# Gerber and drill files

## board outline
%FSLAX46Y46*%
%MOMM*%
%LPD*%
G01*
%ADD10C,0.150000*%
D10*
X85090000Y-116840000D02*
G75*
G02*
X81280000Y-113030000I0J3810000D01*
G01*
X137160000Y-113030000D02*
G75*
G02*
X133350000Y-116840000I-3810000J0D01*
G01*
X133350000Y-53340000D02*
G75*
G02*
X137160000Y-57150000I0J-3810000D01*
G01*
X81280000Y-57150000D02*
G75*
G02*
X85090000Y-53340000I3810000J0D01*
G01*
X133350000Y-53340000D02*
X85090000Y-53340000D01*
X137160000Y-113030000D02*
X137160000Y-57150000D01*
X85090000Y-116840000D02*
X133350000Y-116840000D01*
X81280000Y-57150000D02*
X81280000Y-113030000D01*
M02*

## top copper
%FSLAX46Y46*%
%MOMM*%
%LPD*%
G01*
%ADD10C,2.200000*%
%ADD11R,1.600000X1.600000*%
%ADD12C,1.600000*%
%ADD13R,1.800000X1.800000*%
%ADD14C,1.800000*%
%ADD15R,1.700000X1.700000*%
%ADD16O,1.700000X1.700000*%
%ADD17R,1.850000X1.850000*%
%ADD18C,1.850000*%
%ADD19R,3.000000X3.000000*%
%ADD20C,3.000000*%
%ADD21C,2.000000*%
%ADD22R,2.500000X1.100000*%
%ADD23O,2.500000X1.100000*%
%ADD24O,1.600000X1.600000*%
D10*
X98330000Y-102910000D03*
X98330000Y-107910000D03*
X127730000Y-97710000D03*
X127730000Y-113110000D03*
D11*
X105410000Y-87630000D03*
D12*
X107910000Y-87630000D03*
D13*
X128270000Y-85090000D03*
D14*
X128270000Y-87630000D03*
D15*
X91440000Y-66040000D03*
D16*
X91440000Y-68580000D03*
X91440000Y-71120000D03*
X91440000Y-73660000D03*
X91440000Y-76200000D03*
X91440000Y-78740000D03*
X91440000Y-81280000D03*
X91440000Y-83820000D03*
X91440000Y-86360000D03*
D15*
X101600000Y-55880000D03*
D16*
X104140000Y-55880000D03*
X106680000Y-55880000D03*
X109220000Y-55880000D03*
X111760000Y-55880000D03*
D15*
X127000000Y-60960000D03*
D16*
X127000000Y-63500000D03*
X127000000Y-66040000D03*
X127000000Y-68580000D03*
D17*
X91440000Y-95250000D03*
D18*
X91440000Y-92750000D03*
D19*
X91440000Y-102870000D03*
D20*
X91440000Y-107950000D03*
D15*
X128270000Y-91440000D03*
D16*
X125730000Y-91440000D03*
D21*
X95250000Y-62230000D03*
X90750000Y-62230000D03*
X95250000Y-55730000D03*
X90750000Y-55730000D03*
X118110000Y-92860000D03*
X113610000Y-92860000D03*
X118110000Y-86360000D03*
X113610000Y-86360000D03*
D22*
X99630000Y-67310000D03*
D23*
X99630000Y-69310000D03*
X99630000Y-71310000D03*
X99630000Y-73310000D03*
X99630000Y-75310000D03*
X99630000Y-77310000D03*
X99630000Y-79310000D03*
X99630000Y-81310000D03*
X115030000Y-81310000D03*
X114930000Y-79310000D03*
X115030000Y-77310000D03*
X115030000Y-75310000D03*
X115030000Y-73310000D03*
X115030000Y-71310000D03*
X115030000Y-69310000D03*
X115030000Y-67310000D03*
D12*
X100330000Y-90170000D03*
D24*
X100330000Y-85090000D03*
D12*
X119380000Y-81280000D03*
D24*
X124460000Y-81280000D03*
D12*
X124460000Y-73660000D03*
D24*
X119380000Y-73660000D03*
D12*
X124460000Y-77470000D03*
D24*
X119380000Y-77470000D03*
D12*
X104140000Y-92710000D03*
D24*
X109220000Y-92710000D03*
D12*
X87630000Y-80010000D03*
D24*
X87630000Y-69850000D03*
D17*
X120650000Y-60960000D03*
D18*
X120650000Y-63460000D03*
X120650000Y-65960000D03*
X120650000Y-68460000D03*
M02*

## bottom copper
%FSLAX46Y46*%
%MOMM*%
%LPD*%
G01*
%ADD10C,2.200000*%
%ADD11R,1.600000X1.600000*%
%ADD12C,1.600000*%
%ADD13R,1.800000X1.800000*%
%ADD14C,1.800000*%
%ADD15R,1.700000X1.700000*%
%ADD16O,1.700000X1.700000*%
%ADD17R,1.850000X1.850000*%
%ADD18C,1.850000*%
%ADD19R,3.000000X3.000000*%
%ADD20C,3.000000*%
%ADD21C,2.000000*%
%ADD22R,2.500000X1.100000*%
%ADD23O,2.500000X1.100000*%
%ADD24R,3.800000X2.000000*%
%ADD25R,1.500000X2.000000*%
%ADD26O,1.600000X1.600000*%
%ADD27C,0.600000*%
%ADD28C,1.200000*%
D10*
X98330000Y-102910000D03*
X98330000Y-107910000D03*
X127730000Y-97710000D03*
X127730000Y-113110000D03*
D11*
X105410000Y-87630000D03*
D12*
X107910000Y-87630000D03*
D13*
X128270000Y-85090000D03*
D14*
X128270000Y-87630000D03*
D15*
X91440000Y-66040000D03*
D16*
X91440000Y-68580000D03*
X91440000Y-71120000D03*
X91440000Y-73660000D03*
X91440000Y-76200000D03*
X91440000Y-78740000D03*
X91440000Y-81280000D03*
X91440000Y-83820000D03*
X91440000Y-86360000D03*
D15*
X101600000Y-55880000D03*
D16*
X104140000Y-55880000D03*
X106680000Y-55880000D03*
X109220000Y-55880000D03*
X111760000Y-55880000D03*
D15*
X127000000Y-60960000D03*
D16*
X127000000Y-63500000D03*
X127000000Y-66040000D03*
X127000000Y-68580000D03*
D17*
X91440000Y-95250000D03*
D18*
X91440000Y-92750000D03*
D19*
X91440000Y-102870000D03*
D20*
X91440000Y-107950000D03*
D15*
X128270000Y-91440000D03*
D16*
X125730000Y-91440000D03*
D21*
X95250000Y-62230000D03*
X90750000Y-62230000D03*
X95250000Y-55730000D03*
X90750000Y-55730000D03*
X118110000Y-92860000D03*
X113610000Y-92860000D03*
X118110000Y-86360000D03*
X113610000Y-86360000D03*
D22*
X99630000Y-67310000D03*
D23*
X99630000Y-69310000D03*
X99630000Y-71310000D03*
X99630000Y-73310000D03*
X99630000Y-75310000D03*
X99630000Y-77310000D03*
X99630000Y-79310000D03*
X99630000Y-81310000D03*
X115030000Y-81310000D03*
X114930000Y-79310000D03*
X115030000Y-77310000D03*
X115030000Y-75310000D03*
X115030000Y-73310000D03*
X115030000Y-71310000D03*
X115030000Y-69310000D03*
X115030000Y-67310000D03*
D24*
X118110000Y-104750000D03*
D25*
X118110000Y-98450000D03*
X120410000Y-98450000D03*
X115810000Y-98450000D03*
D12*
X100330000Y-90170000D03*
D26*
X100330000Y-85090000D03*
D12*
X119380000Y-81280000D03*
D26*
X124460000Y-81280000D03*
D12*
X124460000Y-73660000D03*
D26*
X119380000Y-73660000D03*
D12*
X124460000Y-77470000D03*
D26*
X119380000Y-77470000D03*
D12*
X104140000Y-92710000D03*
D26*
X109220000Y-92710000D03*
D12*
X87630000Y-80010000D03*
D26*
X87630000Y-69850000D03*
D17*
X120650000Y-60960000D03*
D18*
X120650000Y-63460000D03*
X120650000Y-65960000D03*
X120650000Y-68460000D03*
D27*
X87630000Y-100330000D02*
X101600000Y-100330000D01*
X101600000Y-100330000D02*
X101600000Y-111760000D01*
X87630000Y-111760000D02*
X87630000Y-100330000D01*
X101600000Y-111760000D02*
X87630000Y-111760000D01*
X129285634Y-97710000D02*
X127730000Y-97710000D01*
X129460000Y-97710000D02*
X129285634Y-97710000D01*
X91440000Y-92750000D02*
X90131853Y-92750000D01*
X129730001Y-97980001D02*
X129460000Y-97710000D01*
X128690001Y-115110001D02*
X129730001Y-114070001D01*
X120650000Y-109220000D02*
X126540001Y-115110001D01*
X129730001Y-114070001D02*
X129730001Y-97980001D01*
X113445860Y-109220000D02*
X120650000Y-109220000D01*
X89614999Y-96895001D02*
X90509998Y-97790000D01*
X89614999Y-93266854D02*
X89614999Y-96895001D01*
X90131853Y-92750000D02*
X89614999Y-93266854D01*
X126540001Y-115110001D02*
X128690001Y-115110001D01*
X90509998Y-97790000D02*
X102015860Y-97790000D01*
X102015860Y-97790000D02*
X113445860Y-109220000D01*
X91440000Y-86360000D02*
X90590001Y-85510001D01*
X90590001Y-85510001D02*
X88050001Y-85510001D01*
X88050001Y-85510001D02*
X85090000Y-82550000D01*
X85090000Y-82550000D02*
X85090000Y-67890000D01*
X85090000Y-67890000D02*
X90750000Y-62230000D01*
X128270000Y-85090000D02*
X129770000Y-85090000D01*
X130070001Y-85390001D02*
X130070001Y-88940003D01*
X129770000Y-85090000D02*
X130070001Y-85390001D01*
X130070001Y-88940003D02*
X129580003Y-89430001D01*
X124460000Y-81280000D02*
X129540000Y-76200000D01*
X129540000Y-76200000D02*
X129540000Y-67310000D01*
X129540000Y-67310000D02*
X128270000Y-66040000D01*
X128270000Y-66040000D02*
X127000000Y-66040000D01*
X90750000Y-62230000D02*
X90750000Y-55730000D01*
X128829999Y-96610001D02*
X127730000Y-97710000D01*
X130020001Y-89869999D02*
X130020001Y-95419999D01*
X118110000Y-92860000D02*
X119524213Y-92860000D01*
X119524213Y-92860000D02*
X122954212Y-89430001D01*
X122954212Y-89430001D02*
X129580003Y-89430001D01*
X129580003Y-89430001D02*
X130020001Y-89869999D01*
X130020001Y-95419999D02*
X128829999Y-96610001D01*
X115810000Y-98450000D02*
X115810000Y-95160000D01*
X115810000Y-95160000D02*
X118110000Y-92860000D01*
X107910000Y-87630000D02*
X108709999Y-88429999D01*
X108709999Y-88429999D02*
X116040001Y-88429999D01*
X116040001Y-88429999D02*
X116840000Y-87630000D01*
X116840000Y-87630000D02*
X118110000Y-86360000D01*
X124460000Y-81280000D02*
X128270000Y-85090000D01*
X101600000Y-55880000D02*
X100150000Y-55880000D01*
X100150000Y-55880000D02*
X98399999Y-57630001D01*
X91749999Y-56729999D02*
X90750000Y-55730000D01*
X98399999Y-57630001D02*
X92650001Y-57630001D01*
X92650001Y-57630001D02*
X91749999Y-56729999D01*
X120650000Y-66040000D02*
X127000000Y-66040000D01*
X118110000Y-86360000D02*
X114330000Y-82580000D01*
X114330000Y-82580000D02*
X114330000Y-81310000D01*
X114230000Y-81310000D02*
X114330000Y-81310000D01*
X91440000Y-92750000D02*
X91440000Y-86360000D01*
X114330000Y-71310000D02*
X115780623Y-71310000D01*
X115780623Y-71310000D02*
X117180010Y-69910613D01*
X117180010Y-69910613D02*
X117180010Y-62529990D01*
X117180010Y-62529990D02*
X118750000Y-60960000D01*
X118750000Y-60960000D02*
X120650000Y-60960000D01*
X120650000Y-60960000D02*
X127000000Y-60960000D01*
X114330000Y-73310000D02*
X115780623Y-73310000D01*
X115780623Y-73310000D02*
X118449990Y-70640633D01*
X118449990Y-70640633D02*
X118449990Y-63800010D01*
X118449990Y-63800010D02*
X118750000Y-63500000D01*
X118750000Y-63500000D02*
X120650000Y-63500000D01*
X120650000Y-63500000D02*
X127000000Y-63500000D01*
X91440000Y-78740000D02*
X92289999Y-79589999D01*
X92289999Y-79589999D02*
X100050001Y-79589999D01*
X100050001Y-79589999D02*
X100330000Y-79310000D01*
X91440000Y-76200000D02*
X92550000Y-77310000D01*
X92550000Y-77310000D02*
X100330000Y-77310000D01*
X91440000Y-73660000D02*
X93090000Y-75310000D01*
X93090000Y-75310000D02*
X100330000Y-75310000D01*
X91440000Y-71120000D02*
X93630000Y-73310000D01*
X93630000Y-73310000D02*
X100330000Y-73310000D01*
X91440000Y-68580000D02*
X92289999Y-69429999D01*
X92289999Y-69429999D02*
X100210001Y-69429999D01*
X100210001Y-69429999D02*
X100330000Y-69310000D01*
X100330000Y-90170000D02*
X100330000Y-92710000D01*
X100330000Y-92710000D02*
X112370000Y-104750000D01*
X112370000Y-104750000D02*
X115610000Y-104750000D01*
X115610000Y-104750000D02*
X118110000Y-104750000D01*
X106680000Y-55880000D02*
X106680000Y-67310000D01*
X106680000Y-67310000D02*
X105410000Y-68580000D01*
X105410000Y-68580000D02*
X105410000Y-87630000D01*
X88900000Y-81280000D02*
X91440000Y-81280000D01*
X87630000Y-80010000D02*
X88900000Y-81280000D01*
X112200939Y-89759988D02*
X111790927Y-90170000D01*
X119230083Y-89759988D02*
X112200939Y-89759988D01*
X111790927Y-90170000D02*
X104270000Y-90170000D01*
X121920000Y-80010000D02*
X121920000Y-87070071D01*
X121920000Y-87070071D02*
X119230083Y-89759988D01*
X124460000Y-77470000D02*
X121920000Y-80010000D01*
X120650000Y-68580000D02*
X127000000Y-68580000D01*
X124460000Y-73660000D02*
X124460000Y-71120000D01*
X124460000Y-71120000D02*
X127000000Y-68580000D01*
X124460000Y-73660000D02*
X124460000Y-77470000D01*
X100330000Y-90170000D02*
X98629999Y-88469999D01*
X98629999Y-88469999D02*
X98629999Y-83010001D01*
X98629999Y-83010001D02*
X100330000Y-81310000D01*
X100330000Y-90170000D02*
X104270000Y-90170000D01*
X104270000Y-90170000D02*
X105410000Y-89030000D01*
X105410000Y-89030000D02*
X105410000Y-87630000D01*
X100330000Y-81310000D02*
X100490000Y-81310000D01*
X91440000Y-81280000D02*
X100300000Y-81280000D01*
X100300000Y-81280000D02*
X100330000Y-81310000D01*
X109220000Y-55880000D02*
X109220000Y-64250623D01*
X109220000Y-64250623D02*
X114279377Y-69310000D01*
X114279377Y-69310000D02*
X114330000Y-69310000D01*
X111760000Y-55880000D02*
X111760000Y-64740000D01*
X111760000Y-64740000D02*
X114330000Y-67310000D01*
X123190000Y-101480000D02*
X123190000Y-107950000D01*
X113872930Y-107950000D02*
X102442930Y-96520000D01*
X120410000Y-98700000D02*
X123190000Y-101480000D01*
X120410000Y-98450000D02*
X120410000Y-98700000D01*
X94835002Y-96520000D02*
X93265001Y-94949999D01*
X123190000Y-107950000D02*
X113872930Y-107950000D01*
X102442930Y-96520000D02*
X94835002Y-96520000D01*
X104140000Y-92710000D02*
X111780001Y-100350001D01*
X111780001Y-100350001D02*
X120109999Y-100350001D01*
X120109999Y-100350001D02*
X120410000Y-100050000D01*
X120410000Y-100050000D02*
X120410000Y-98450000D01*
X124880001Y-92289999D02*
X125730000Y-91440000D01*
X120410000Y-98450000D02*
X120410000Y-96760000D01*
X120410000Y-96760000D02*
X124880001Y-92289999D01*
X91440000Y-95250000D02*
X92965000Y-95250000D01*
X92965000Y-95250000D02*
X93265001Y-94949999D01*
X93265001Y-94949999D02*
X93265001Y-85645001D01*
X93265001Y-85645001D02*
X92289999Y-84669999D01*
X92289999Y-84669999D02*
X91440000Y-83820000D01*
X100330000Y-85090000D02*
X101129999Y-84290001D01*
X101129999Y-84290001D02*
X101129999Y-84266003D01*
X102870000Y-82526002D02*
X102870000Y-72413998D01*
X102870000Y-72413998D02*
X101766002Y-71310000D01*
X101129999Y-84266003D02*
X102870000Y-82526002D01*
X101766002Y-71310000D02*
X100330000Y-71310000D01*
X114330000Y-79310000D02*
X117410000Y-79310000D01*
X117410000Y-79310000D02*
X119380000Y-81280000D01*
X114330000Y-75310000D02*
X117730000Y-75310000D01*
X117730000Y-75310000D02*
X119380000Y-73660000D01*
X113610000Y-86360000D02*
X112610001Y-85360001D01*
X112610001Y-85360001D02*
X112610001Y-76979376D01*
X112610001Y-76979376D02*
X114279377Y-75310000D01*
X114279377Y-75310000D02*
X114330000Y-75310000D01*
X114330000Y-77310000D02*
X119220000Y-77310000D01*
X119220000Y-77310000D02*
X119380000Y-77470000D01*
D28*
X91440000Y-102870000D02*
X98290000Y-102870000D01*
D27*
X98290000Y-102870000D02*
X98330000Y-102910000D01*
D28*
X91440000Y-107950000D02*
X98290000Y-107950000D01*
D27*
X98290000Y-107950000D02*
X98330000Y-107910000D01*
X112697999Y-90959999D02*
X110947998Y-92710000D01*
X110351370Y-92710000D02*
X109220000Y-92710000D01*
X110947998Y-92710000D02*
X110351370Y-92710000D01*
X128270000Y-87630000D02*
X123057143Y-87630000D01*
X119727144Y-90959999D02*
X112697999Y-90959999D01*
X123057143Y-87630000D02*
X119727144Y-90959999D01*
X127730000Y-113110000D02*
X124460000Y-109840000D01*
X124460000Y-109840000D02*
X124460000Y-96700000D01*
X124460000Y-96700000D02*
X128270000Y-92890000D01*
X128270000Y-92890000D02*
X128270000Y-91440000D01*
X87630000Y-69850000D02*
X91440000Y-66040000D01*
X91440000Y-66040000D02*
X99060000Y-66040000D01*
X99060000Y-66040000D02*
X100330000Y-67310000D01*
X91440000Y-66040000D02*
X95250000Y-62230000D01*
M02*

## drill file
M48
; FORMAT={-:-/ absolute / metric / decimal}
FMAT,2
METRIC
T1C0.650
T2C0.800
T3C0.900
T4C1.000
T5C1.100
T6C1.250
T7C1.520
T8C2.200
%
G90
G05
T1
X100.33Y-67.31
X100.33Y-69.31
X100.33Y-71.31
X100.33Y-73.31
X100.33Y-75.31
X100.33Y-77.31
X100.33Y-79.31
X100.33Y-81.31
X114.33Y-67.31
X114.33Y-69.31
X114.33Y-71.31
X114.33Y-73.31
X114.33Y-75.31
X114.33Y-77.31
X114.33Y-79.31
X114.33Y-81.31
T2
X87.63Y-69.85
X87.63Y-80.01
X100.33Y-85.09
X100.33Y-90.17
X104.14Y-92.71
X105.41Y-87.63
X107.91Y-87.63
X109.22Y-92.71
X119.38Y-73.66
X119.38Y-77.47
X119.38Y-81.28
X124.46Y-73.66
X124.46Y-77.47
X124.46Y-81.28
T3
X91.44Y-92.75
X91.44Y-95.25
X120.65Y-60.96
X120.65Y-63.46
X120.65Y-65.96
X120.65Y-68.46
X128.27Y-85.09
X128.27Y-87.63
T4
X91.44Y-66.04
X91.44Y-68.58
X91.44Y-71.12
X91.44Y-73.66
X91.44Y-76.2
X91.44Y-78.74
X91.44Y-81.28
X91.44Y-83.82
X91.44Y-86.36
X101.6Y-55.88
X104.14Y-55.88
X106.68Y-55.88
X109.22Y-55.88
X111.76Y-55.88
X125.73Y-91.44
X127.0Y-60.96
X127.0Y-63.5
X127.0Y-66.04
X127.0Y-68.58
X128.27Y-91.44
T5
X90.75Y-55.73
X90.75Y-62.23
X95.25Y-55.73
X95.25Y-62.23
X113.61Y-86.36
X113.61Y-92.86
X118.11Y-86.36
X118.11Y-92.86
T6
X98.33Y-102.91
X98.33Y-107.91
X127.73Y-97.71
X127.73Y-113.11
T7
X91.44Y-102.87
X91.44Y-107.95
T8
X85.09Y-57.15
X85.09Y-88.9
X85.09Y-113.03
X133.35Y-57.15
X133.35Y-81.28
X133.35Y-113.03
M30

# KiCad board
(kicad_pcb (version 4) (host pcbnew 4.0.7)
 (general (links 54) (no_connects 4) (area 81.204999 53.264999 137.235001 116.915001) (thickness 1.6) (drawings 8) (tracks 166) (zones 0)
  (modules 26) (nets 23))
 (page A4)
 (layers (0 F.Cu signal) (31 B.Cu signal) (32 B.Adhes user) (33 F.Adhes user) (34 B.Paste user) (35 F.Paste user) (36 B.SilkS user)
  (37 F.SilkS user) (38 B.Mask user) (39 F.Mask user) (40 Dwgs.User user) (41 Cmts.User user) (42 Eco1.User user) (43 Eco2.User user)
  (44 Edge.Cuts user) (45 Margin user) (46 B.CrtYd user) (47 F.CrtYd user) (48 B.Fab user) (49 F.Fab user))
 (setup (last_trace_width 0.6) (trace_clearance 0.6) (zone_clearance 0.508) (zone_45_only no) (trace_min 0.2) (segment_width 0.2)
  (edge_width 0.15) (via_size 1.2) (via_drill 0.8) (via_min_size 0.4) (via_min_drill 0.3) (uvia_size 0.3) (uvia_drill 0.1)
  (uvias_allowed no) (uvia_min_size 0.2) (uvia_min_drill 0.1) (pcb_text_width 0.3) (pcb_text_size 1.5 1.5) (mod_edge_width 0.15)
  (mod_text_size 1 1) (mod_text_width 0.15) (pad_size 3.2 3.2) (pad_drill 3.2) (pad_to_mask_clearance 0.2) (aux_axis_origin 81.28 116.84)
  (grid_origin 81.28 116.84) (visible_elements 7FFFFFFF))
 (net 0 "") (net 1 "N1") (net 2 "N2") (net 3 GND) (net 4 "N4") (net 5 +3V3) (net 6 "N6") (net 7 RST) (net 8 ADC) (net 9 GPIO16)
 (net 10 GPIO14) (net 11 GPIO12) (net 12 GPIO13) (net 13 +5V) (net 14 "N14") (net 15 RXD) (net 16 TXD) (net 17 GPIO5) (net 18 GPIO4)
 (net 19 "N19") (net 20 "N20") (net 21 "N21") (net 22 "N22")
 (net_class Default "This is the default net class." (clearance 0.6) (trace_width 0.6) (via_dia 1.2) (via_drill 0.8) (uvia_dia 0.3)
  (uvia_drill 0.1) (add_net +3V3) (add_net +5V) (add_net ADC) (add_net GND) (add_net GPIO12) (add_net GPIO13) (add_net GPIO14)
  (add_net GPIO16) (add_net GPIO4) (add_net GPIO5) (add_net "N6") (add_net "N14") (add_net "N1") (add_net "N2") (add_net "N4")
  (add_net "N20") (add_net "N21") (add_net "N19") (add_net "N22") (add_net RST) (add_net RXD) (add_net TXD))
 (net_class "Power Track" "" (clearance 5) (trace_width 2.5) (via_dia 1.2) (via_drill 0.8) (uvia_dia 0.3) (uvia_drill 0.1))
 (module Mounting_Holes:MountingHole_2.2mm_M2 (layer F.Cu) (at 85.09 88.9)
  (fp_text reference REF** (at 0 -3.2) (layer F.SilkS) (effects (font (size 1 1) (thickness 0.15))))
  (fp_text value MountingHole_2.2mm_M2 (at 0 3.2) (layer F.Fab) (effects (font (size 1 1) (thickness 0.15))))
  (pad 1 np_thru_hole circle (at 0 0) (size 2.2 2.2) (drill 2.2) (layers *.Cu *.Mask)))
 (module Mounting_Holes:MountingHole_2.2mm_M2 (layer F.Cu) (at 133.35 81.28)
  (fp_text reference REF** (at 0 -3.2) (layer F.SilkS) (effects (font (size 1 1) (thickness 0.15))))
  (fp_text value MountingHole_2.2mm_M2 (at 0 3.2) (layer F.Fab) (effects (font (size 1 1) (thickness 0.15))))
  (pad 1 np_thru_hole circle (at 0 0) (size 2.2 2.2) (drill 2.2) (layers *.Cu *.Mask)))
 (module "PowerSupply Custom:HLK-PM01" (layer F.Cu) (at 113.03 105.41)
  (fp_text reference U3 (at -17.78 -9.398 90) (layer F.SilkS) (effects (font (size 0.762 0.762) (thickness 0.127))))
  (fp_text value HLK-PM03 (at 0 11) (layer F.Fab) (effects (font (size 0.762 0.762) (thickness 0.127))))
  (pad 1 thru_hole circle (at -14.7 -2.5) (size 2.2 2.2) (drill 1.25) (layers *.Cu *.Mask) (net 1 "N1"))
  (pad 2 thru_hole circle (at -14.7 2.5) (size 2.2 2.2) (drill 1.25) (layers *.Cu *.Mask) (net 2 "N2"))
  (pad 3 thru_hole circle (at 14.7 -7.7) (size 2.2 2.2) (drill 1.25) (layers *.Cu *.Mask) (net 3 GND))
  (pad 4 thru_hole circle (at 14.7 7.7) (size 2.2 2.2) (drill 1.25) (layers *.Cu *.Mask) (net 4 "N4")))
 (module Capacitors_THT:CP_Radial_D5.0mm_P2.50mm (layer F.Cu) (at 105.41 87.63)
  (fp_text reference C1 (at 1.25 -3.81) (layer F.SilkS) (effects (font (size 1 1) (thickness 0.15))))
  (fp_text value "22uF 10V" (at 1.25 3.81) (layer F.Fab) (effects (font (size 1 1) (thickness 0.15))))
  (pad 1 thru_hole rect (at 0 0) (size 1.6 1.6) (drill 0.8) (layers *.Cu *.Mask) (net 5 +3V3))
  (pad 2 thru_hole circle (at 2.5 0) (size 1.6 1.6) (drill 0.8) (layers *.Cu *.Mask) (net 3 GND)))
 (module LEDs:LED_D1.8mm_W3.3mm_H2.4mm (layer F.Cu) (at 128.27 85.09 270)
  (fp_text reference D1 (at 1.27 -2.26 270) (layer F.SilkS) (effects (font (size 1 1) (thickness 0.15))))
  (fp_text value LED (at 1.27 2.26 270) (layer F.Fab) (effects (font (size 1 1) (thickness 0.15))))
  (pad 1 thru_hole rect (at 0 0 270) (size 1.8 1.8) (drill 0.9) (layers *.Cu *.Mask) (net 3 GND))
  (pad 2 thru_hole circle (at 2.54 0 270) (size 1.8 1.8) (drill 0.9) (layers *.Cu *.Mask) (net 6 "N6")))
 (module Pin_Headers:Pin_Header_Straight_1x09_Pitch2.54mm (layer F.Cu) (at 91.44 66.04)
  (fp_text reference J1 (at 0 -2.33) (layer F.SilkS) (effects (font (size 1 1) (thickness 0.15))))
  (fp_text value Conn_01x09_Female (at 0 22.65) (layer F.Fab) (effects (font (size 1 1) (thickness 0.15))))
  (pad 1 thru_hole rect (at 0 0) (size 1.7 1.7) (drill 1) (layers *.Cu *.Mask) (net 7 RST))
  (pad 2 thru_hole oval (at 0 2.54) (size 1.7 1.7) (drill 1) (layers *.Cu *.Mask) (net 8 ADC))
  (pad 3 thru_hole oval (at 0 5.08) (size 1.7 1.7) (drill 1) (layers *.Cu *.Mask) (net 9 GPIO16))
  (pad 4 thru_hole oval (at 0 7.62) (size 1.7 1.7) (drill 1) (layers *.Cu *.Mask) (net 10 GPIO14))
  (pad 5 thru_hole oval (at 0 10.16) (size 1.7 1.7) (drill 1) (layers *.Cu *.Mask) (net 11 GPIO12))
  (pad 6 thru_hole oval (at 0 12.7) (size 1.7 1.7) (drill 1) (layers *.Cu *.Mask) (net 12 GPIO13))
  (pad 7 thru_hole oval (at 0 15.24) (size 1.7 1.7) (drill 1) (layers *.Cu *.Mask) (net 5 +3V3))
  (pad 8 thru_hole oval (at 0 17.78) (size 1.7 1.7) (drill 1) (layers *.Cu *.Mask) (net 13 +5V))
  (pad 9 thru_hole oval (at 0 20.32) (size 1.7 1.7) (drill 1) (layers *.Cu *.Mask) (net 3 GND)))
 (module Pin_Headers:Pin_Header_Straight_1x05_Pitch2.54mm (layer F.Cu) (at 101.6 55.88 90)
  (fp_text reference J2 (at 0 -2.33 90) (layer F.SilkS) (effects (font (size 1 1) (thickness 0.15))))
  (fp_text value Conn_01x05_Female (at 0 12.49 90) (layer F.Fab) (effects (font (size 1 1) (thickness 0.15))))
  (pad 1 thru_hole rect (at 0 0 90) (size 1.7 1.7) (drill 1) (layers *.Cu *.Mask) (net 3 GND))
  (pad 2 thru_hole oval (at 0 2.54 90) (size 1.7 1.7) (drill 1) (layers *.Cu *.Mask) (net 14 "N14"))
  (pad 3 thru_hole oval (at 0 5.08 90) (size 1.7 1.7) (drill 1) (layers *.Cu *.Mask) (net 5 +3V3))
  (pad 4 thru_hole oval (at 0 7.62 90) (size 1.7 1.7) (drill 1) (layers *.Cu *.Mask) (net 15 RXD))
  (pad 5 thru_hole oval (at 0 10.16 90) (size 1.7 1.7) (drill 1) (layers *.Cu *.Mask) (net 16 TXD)))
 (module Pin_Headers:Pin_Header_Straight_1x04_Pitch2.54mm (layer F.Cu) (at 127 60.96)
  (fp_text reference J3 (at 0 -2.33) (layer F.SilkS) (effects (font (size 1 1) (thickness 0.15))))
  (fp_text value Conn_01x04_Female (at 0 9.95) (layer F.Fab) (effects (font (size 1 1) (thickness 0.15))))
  (pad 1 thru_hole rect (at 0 0) (size 1.7 1.7) (drill 1) (layers *.Cu *.Mask) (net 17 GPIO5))
  (pad 2 thru_hole oval (at 0 2.54) (size 1.7 1.7) (drill 1) (layers *.Cu *.Mask) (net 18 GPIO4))
  (pad 3 thru_hole oval (at 0 5.08) (size 1.7 1.7) (drill 1) (layers *.Cu *.Mask) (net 3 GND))
  (pad 4 thru_hole oval (at 0 7.62) (size 1.7 1.7) (drill 1) (layers *.Cu *.Mask) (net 5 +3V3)))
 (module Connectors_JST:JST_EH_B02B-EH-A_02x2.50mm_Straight (layer F.Cu) (at 91.44 95.25 90)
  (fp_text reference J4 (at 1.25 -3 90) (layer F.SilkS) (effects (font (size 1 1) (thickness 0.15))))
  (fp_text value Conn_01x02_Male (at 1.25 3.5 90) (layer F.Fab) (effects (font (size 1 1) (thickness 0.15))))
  (pad 1 thru_hole rect (at 0 0 90) (size 1.85 1.85) (drill 0.9) (layers *.Cu *.Mask) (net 13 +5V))
  (pad 2 thru_hole circle (at 2.5 0 90) (size 1.85 1.85) (drill 0.9) (layers *.Cu *.Mask) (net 3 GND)))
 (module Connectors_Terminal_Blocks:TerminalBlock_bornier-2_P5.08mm (layer F.Cu) (at 91.44 102.87 270)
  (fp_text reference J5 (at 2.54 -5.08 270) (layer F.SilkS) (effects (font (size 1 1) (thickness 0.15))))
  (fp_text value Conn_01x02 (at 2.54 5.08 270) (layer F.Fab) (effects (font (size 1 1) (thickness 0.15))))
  (pad 1 thru_hole rect (at 0 0 270) (size 3 3) (drill 1.52) (layers *.Cu *.Mask) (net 1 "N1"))
  (pad 2 thru_hole circle (at 5.08 0 270) (size 3 3) (drill 1.52) (layers *.Cu *.Mask) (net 2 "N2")))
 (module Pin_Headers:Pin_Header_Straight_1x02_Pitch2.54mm (layer F.Cu) (at 128.27 91.44 270)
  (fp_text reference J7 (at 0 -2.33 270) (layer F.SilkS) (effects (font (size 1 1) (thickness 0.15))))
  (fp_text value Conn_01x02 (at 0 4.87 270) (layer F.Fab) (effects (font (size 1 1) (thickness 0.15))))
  (pad 1 thru_hole rect (at 0 0 270) (size 1.7 1.7) (drill 1) (layers *.Cu *.Mask) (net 4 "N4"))
  (pad 2 thru_hole oval (at 0 2.54 270) (size 1.7 1.7) (drill 1) (layers *.Cu *.Mask) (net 13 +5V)))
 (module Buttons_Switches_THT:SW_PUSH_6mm (layer F.Cu) (at 90.75 62.23 90)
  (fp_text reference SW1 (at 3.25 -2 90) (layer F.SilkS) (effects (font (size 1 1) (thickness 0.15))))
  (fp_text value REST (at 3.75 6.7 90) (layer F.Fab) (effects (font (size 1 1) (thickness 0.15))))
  (pad 2 thru_hole circle (at 0 4.5 180) (size 2 2) (drill 1.1) (layers *.Cu *.Mask) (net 7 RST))
  (pad 1 thru_hole circle (at 0 0 180) (size 2 2) (drill 1.1) (layers *.Cu *.Mask) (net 3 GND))
  (pad 2 thru_hole circle (at 6.5 4.5 180) (size 2 2) (drill 1.1) (layers *.Cu *.Mask) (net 7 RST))
  (pad 1 thru_hole circle (at 6.5 0 180) (size 2 2) (drill 1.1) (layers *.Cu *.Mask) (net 3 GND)))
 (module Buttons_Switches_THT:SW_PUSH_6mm (layer F.Cu) (at 113.61 92.86 90)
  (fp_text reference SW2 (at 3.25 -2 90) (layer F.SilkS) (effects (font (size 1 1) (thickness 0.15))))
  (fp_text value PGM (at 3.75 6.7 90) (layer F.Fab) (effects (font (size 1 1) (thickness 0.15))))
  (pad 2 thru_hole circle (at 0 4.5 180) (size 2 2) (drill 1.1) (layers *.Cu *.Mask) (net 3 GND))
  (pad 1 thru_hole circle (at 0 0 180) (size 2 2) (drill 1.1) (layers *.Cu *.Mask) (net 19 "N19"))
  (pad 2 thru_hole circle (at 6.5 4.5 180) (size 2 2) (drill 1.1) (layers *.Cu *.Mask) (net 3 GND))
  (pad 1 thru_hole circle (at 6.5 0 180) (size 2 2) (drill 1.1) (layers *.Cu *.Mask) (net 19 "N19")))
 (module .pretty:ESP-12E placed (layer F.Cu) (at 100.33 67.31)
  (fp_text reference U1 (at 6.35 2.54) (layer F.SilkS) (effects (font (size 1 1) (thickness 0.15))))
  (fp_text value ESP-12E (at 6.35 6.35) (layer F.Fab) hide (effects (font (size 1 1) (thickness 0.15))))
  (pad 1 thru_hole rect (at 0 0) (size 2.5 1.1) (drill 0.65 (offset -0.7 0)) (layers *.Cu *.Mask F.SilkS) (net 7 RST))
  (pad 2 thru_hole oval (at 0 2) (size 2.5 1.1) (drill 0.65 (offset -0.7 0)) (layers *.Cu *.Mask F.SilkS) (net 8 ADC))
  (pad 3 thru_hole oval (at 0 4) (size 2.5 1.1) (drill 0.65 (offset -0.7 0)) (layers *.Cu *.Mask F.SilkS) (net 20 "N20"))
  (pad 4 thru_hole oval (at 0 6) (size 2.5 1.1) (drill 0.65 (offset -0.7 0)) (layers *.Cu *.Mask F.SilkS) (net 9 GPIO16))
  (pad 5 thru_hole oval (at 0 8) (size 2.5 1.1) (drill 0.65 (offset -0.7 0)) (layers *.Cu *.Mask F.SilkS) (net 10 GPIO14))
  (pad 6 thru_hole oval (at 0 10) (size 2.5 1.1) (drill 0.65 (offset -0.7 0)) (layers *.Cu *.Mask F.SilkS) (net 11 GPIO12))
  (pad 7 thru_hole oval (at 0 12) (size 2.5 1.1) (drill 0.65 (offset -0.7 0)) (layers *.Cu *.Mask F.SilkS) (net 12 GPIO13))
  (pad 8 thru_hole oval (at 0 14) (size 2.5 1.1) (drill 0.65 (offset -0.7 0)) (layers *.Cu *.Mask F.SilkS) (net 5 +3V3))
  (pad 9 thru_hole oval (at 14 14) (size 2.5 1.1) (drill 0.65 (offset 0.7 0)) (layers *.Cu *.Mask F.SilkS) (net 3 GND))
  (pad 10 thru_hole oval (at 14 12) (size 2.5 1.1) (drill 0.65 (offset 0.6 0)) (layers *.Cu *.Mask F.SilkS) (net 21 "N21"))
  (pad 11 thru_hole oval (at 14 10) (size 2.5 1.1) (drill 0.65 (offset 0.7 0)) (layers *.Cu *.Mask F.SilkS) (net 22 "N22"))
  (pad 12 thru_hole oval (at 14 8) (size 2.5 1.1) (drill 0.65 (offset 0.7 0)) (layers *.Cu *.Mask F.SilkS) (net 19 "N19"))
  (pad 13 thru_hole oval (at 14 6) (size 2.5 1.1) (drill 0.65 (offset 0.7 0)) (layers *.Cu *.Mask F.SilkS) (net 18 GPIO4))
  (pad 14 thru_hole oval (at 14 4) (size 2.5 1.1) (drill 0.65 (offset 0.7 0)) (layers *.Cu *.Mask F.SilkS) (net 17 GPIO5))
  (pad 15 thru_hole oval (at 14 2) (size 2.5 1.1) (drill 0.65 (offset 0.7 0)) (layers *.Cu *.Mask F.SilkS) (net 15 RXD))
  (pad 16 thru_hole oval (at 14 0) (size 2.5 1.1) (drill 0.65 (offset 0.7 0)) (layers *.Cu *.Mask F.SilkS) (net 16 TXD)))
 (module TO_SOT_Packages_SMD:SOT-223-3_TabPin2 (layer B.Cu) (at 118.11 101.6 270)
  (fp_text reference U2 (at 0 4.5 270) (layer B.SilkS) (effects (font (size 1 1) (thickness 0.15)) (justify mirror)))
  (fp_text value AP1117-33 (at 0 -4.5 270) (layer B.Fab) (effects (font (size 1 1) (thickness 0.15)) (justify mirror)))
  (pad 2 smd rect (at 3.15 0 270) (size 2 3.8) (layers B.Cu B.Paste B.Mask) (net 5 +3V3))
  (pad 2 smd rect (at -3.15 0 270) (size 2 1.5) (layers B.Cu B.Paste B.Mask) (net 5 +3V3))
  (pad 3 smd rect (at -3.15 -2.3 270) (size 2 1.5) (layers B.Cu B.Paste B.Mask) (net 13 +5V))
  (pad 1 smd rect (at -3.15 2.3 270) (size 2 1.5) (layers B.Cu B.Paste B.Mask) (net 3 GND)))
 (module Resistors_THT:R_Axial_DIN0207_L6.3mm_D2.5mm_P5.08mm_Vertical (layer F.Cu) (at 100.33 90.17 90)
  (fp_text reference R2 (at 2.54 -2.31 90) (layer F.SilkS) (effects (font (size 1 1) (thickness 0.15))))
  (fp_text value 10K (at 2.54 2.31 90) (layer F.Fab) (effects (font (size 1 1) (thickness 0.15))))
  (pad 1 thru_hole circle (at 0 0 90) (size 1.6 1.6) (drill 0.8) (layers *.Cu *.Mask) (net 5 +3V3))
  (pad 2 thru_hole oval (at 5.08 0 90) (size 1.6 1.6) (drill 0.8) (layers *.Cu *.Mask) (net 20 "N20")))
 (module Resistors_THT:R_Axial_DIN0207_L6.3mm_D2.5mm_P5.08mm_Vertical (layer F.Cu) (at 119.38 81.28)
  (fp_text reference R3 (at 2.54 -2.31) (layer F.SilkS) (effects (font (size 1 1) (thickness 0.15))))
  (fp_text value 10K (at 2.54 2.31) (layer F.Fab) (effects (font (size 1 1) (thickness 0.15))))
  (pad 1 thru_hole circle (at 0 0) (size 1.6 1.6) (drill 0.8) (layers *.Cu *.Mask) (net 21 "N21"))
  (pad 2 thru_hole oval (at 5.08 0) (size 1.6 1.6) (drill 0.8) (layers *.Cu *.Mask) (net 3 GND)))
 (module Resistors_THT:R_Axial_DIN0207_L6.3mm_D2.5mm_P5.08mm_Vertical (layer F.Cu) (at 124.46 73.66 180)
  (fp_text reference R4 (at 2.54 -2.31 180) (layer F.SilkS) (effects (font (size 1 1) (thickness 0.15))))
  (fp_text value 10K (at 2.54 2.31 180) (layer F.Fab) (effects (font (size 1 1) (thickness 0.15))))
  (pad 1 thru_hole circle (at 0 0 180) (size 1.6 1.6) (drill 0.8) (layers *.Cu *.Mask) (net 5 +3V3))
  (pad 2 thru_hole oval (at 5.08 0 180) (size 1.6 1.6) (drill 0.8) (layers *.Cu *.Mask) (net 19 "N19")))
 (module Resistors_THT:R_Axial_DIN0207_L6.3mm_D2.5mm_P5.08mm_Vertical (layer F.Cu) (at 124.46 77.47 180)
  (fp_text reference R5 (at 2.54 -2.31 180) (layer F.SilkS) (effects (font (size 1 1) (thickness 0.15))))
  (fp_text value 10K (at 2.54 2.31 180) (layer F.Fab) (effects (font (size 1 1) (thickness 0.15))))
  (pad 1 thru_hole circle (at 0 0 180) (size 1.6 1.6) (drill 0.8) (layers *.Cu *.Mask) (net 5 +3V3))
  (pad 2 thru_hole oval (at 5.08 0 180) (size 1.6 1.6) (drill 0.8) (layers *.Cu *.Mask) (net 22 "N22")))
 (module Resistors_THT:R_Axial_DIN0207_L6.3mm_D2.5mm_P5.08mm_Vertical (layer F.Cu) (at 104.14 92.71)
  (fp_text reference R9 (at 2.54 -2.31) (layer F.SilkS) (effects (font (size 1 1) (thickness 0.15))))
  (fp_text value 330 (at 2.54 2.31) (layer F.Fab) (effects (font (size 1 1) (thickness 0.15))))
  (pad 1 thru_hole circle (at 0 0) (size 1.6 1.6) (drill 0.8) (layers *.Cu *.Mask) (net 13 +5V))
  (pad 2 thru_hole oval (at 5.08 0) (size 1.6 1.6) (drill 0.8) (layers *.Cu *.Mask) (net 6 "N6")))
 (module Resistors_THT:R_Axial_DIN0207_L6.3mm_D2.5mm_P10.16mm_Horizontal (layer F.Cu) (at 87.63 80.01 90)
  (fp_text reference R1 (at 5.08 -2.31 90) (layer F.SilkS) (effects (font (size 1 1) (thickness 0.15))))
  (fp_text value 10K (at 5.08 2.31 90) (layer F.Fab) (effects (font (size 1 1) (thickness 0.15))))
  (pad 1 thru_hole circle (at 0 0 90) (size 1.6 1.6) (drill 0.8) (layers *.Cu *.Mask) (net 5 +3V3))
  (pad 2 thru_hole oval (at 10.16 0 90) (size 1.6 1.6) (drill 0.8) (layers *.Cu *.Mask) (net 7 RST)))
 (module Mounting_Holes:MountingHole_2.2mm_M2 (layer F.Cu) (at 85.09 57.15)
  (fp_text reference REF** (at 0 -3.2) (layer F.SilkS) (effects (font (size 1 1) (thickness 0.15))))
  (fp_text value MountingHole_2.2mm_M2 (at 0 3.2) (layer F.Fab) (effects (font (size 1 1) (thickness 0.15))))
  (pad 1 np_thru_hole circle (at 0 0) (size 2.2 2.2) (drill 2.2) (layers *.Cu *.Mask)))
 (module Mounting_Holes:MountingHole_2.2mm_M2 (layer F.Cu) (at 133.35 57.15)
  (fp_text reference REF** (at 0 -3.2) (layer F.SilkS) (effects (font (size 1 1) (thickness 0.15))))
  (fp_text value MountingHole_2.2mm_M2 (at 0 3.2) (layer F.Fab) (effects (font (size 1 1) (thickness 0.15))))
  (pad 1 np_thru_hole circle (at 0 0) (size 2.2 2.2) (drill 2.2) (layers *.Cu *.Mask)))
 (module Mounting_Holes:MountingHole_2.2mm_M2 (layer F.Cu) (at 133.35 113.03)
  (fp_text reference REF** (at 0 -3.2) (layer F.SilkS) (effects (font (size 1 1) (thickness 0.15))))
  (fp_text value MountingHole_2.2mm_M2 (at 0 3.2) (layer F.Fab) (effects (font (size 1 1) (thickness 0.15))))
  (pad 1 np_thru_hole circle (at 0 0) (size 2.2 2.2) (drill 2.2) (layers *.Cu *.Mask)))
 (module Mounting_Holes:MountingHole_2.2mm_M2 (layer F.Cu) (at 85.09 113.03)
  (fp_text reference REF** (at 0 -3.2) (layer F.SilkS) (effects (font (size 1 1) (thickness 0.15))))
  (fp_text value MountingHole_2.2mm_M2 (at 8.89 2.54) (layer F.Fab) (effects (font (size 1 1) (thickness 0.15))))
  (pad 1 np_thru_hole circle (at 0 0) (size 2.2 2.2) (drill 2.2) (layers *.Cu *.Mask)))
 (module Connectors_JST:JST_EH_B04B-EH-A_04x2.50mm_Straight (layer F.Cu) (at 120.65 60.96 270)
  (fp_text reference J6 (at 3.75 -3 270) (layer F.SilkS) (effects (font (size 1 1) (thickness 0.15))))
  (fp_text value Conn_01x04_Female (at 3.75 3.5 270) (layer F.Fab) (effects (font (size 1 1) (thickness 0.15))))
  (pad 1 thru_hole rect (at 0 0 270) (size 1.85 1.85) (drill 0.9) (layers *.Cu *.Mask) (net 17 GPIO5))
  (pad 2 thru_hole circle (at 2.5 0 270) (size 1.85 1.85) (drill 0.9) (layers *.Cu *.Mask) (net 18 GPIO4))
  (pad 3 thru_hole circle (at 5 0 270) (size 1.85 1.85) (drill 0.9) (layers *.Cu *.Mask) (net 3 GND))
  (pad 4 thru_hole circle (at 7.5 0 270) (size 1.85 1.85) (drill 0.9) (layers *.Cu *.Mask) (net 5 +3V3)))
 (gr_arc (start 85.09 113.03) (end 85.09 116.84) (angle 90) (layer Edge.Cuts) (width 0.15))
 (gr_arc (start 133.35 113.03) (end 137.16 113.03) (angle 90) (layer Edge.Cuts) (width 0.15))
 (gr_arc (start 133.35 57.15) (end 133.35 53.34) (angle 90) (layer Edge.Cuts) (width 0.15))
 (gr_arc (start 85.09 57.15) (end 81.28 57.15) (angle 90) (layer Edge.Cuts) (width 0.15))
 (gr_line (start 133.35 53.34) (end 85.09 53.34) (layer Edge.Cuts) (width 0.15))
 (gr_line (start 137.16 113.03) (end 137.16 57.15) (layer Edge.Cuts) (width 0.15))
 (gr_line (start 85.09 116.84) (end 133.35 116.84) (layer Edge.Cuts) (width 0.15))
 (gr_line (start 81.28 57.15) (end 81.28 113.03) (layer Edge.Cuts) (width 0.15))
 (segment (start 87.63 100.33) (end 101.6 100.33) (width 0.6) (layer B.Cu) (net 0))
 (segment (start 101.6 100.33) (end 101.6 111.76) (width 0.6) (layer B.Cu) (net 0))
 (segment (start 87.63 111.76) (end 87.63 100.33) (width 0.6) (layer B.Cu) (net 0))
 (segment (start 101.6 111.76) (end 87.63 111.76) (width 0.6) (layer B.Cu) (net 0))
 (segment (start 129.285634 97.71) (end 127.73 97.71) (width 0.6) (layer B.Cu) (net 3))
 (segment (start 129.46 97.71) (end 129.285634 97.71) (width 0.6) (layer B.Cu) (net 3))
 (segment (start 91.44 92.75) (end 90.131853 92.75) (width 0.6) (layer B.Cu) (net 3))
 (segment (start 129.730001 97.980001) (end 129.46 97.71) (width 0.6) (layer B.Cu) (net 3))
 (segment (start 128.690001 115.110001) (end 129.730001 114.070001) (width 0.6) (layer B.Cu) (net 3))
 (segment (start 120.65 109.22) (end 126.540001 115.110001) (width 0.6) (layer B.Cu) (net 3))
 (segment (start 129.730001 114.070001) (end 129.730001 97.980001) (width 0.6) (layer B.Cu) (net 3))
 (segment (start 113.44586 109.22) (end 120.65 109.22) (width 0.6) (layer B.Cu) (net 3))
 (segment (start 89.614999 96.895001) (end 90.509998 97.79) (width 0.6) (layer B.Cu) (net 3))
 (segment (start 89.614999 93.266854) (end 89.614999 96.895001) (width 0.6) (layer B.Cu) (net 3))
 (segment (start 90.131853 92.75) (end 89.614999 93.266854) (width 0.6) (layer B.Cu) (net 3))
 (segment (start 126.540001 115.110001) (end 128.690001 115.110001) (width 0.6) (layer B.Cu) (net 3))
 (segment (start 90.509998 97.79) (end 102.01586 97.79) (width 0.6) (layer B.Cu) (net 3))
 (segment (start 102.01586 97.79) (end 113.44586 109.22) (width 0.6) (layer B.Cu) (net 3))
 (segment (start 91.44 86.36) (end 90.590001 85.510001) (width 0.6) (layer B.Cu) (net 3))
 (segment (start 90.590001 85.510001) (end 88.050001 85.510001) (width 0.6) (layer B.Cu) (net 3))
 (segment (start 88.050001 85.510001) (end 85.09 82.55) (width 0.6) (layer B.Cu) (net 3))
 (segment (start 85.09 82.55) (end 85.09 67.89) (width 0.6) (layer B.Cu) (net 3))
 (segment (start 85.09 67.89) (end 90.75 62.23) (width 0.6) (layer B.Cu) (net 3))
 (segment (start 128.27 85.09) (end 129.77 85.09) (width 0.6) (layer B.Cu) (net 3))
 (segment (start 130.070001 85.390001) (end 130.070001 88.940003) (width 0.6) (layer B.Cu) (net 3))
 (segment (start 129.77 85.09) (end 130.070001 85.390001) (width 0.6) (layer B.Cu) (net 3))
 (segment (start 130.070001 88.940003) (end 129.580003 89.430001) (width 0.6) (layer B.Cu) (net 3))
 (segment (start 124.46 81.28) (end 129.54 76.2) (width 0.6) (layer B.Cu) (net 3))
 (segment (start 129.54 76.2) (end 129.54 67.31) (width 0.6) (layer B.Cu) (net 3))
 (segment (start 129.54 67.31) (end 128.27 66.04) (width 0.6) (layer B.Cu) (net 3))
 (segment (start 128.27 66.04) (end 127 66.04) (width 0.6) (layer B.Cu) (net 3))
 (segment (start 90.75 62.23) (end 90.75 55.73) (width 0.6) (layer B.Cu) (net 3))
 (segment (start 128.829999 96.610001) (end 127.73 97.71) (width 0.6) (layer B.Cu) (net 3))
 (segment (start 130.020001 89.869999) (end 130.020001 95.419999) (width 0.6) (layer B.Cu) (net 3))
 (segment (start 118.11 92.86) (end 119.524213 92.86) (width 0.6) (layer B.Cu) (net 3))
 (segment (start 119.524213 92.86) (end 122.954212 89.430001) (width 0.6) (layer B.Cu) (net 3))
 (segment (start 122.954212 89.430001) (end 129.580003 89.430001) (width 0.6) (layer B.Cu) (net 3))
 (segment (start 129.580003 89.430001) (end 130.020001 89.869999) (width 0.6) (layer B.Cu) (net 3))
 (segment (start 130.020001 95.419999) (end 128.829999 96.610001) (width 0.6) (layer B.Cu) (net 3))
 (segment (start 115.81 98.45) (end 115.81 95.16) (width 0.6) (layer B.Cu) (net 3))
 (segment (start 115.81 95.16) (end 118.11 92.86) (width 0.6) (layer B.Cu) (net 3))
 (segment (start 107.91 87.63) (end 108.709999 88.429999) (width 0.6) (layer B.Cu) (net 3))
 (segment (start 108.709999 88.429999) (end 116.040001 88.429999) (width 0.6) (layer B.Cu) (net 3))
 (segment (start 116.040001 88.429999) (end 116.84 87.63) (width 0.6) (layer B.Cu) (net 3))
 (segment (start 116.84 87.63) (end 118.11 86.36) (width 0.6) (layer B.Cu) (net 3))
 (segment (start 124.46 81.28) (end 128.27 85.09) (width 0.6) (layer B.Cu) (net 3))
 (segment (start 101.6 55.88) (end 100.15 55.88) (width 0.6) (layer B.Cu) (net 3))
 (segment (start 100.15 55.88) (end 98.399999 57.630001) (width 0.6) (layer B.Cu) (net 3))
 (segment (start 91.749999 56.729999) (end 90.75 55.73) (width 0.6) (layer B.Cu) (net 3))
 (segment (start 98.399999 57.630001) (end 92.650001 57.630001) (width 0.6) (layer B.Cu) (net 3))
 (segment (start 92.650001 57.630001) (end 91.749999 56.729999) (width 0.6) (layer B.Cu) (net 3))
 (segment (start 120.65 66.04) (end 127 66.04) (width 0.6) (layer B.Cu) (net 3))
 (segment (start 118.11 86.36) (end 114.33 82.58) (width 0.6) (layer B.Cu) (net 3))
 (segment (start 114.33 82.58) (end 114.33 81.31) (width 0.6) (layer B.Cu) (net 3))
 (segment (start 114.23 81.31) (end 114.33 81.31) (width 0.6) (layer B.Cu) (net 3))
 (segment (start 91.44 92.75) (end 91.44 86.36) (width 0.6) (layer B.Cu) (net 3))
 (segment (start 114.33 71.31) (end 115.780623 71.31) (width 0.6) (layer B.Cu) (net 17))
 (segment (start 115.780623 71.31) (end 117.18001 69.910613) (width 0.6) (layer B.Cu) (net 17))
 (segment (start 117.18001 69.910613) (end 117.18001 62.52999) (width 0.6) (layer B.Cu) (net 17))
 (segment (start 117.18001 62.52999) (end 118.75 60.96) (width 0.6) (layer B.Cu) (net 17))
 (segment (start 118.75 60.96) (end 120.65 60.96) (width 0.6) (layer B.Cu) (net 17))
 (segment (start 120.65 60.96) (end 127 60.96) (width 0.6) (layer B.Cu) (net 17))
 (segment (start 114.33 73.31) (end 115.780623 73.31) (width 0.6) (layer B.Cu) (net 18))
 (segment (start 115.780623 73.31) (end 118.44999 70.640633) (width 0.6) (layer B.Cu) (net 18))
 (segment (start 118.44999 70.640633) (end 118.44999 63.80001) (width 0.6) (layer B.Cu) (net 18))
 (segment (start 118.44999 63.80001) (end 118.75 63.5) (width 0.6) (layer B.Cu) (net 18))
 (segment (start 118.75 63.5) (end 120.65 63.5) (width 0.6) (layer B.Cu) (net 18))
 (segment (start 120.65 63.5) (end 127 63.5) (width 0.6) (layer B.Cu) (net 18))
 (segment (start 91.44 78.74) (end 92.289999 79.589999) (width 0.6) (layer B.Cu) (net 12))
 (segment (start 92.289999 79.589999) (end 100.050001 79.589999) (width 0.6) (layer B.Cu) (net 12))
 (segment (start 100.050001 79.589999) (end 100.33 79.31) (width 0.6) (layer B.Cu) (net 12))
 (segment (start 91.44 76.2) (end 92.55 77.31) (width 0.6) (layer B.Cu) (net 11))
 (segment (start 92.55 77.31) (end 100.33 77.31) (width 0.6) (layer B.Cu) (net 11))
 (segment (start 91.44 73.66) (end 93.09 75.31) (width 0.6) (layer B.Cu) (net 10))
 (segment (start 93.09 75.31) (end 100.33 75.31) (width 0.6) (layer B.Cu) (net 10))
 (segment (start 91.44 71.12) (end 93.63 73.31) (width 0.6) (layer B.Cu) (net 9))
 (segment (start 93.63 73.31) (end 100.33 73.31) (width 0.6) (layer B.Cu) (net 9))
 (segment (start 91.44 68.58) (end 92.289999 69.429999) (width 0.6) (layer B.Cu) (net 8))
 (segment (start 92.289999 69.429999) (end 100.210001 69.429999) (width 0.6) (layer B.Cu) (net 8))
 (segment (start 100.210001 69.429999) (end 100.33 69.31) (width 0.6) (layer B.Cu) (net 8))
 (segment (start 100.33 90.17) (end 100.33 92.71) (width 0.6) (layer B.Cu) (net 5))
 (segment (start 100.33 92.71) (end 112.37 104.75) (width 0.6) (layer B.Cu) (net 5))
 (segment (start 112.37 104.75) (end 115.61 104.75) (width 0.6) (layer B.Cu) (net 5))
 (segment (start 115.61 104.75) (end 118.11 104.75) (width 0.6) (layer B.Cu) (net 5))
 (segment (start 106.68 55.88) (end 106.68 67.31) (width 0.6) (layer B.Cu) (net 5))
 (segment (start 106.68 67.31) (end 105.41 68.58) (width 0.6) (layer B.Cu) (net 5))
 (segment (start 105.41 68.58) (end 105.41 87.63) (width 0.6) (layer B.Cu) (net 5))
 (segment (start 88.9 81.28) (end 91.44 81.28) (width 0.6) (layer B.Cu) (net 5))
 (segment (start 87.63 80.01) (end 88.9 81.28) (width 0.6) (layer B.Cu) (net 5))
 (segment (start 112.200939 89.759988) (end 111.790927 90.17) (width 0.6) (layer B.Cu) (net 5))
 (segment (start 119.230083 89.759988) (end 112.200939 89.759988) (width 0.6) (layer B.Cu) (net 5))
 (segment (start 111.790927 90.17) (end 104.27 90.17) (width 0.6) (layer B.Cu) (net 5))
 (segment (start 121.92 80.01) (end 121.92 87.070071) (width 0.6) (layer B.Cu) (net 5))
 (segment (start 121.92 87.070071) (end 119.230083 89.759988) (width 0.6) (layer B.Cu) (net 5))
 (segment (start 124.46 77.47) (end 121.92 80.01) (width 0.6) (layer B.Cu) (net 5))
 (segment (start 120.65 68.58) (end 127 68.58) (width 0.6) (layer B.Cu) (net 5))
 (segment (start 124.46 73.66) (end 124.46 71.12) (width 0.6) (layer B.Cu) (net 5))
 (segment (start 124.46 71.12) (end 127 68.58) (width 0.6) (layer B.Cu) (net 5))
 (segment (start 124.46 73.66) (end 124.46 77.47) (width 0.6) (layer B.Cu) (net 5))
 (segment (start 100.33 90.17) (end 98.629999 88.469999) (width 0.6) (layer B.Cu) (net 5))
 (segment (start 98.629999 88.469999) (end 98.629999 83.010001) (width 0.6) (layer B.Cu) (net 5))
 (segment (start 98.629999 83.010001) (end 100.33 81.31) (width 0.6) (layer B.Cu) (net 5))
 (segment (start 100.33 90.17) (end 104.27 90.17) (width 0.6) (layer B.Cu) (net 5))
 (segment (start 104.27 90.17) (end 105.41 89.03) (width 0.6) (layer B.Cu) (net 5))
 (segment (start 105.41 89.03) (end 105.41 87.63) (width 0.6) (layer B.Cu) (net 5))
 (segment (start 100.33 81.31) (end 100.49 81.31) (width 0.6) (layer B.Cu) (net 5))
 (segment (start 91.44 81.28) (end 100.3 81.28) (width 0.6) (layer B.Cu) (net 5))
 (segment (start 100.3 81.28) (end 100.33 81.31) (width 0.6) (layer B.Cu) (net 5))
 (segment (start 109.22 55.88) (end 109.22 64.250623) (width 0.6) (layer B.Cu) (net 15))
 (segment (start 109.22 64.250623) (end 114.279377 69.31) (width 0.6) (layer B.Cu) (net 15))
 (segment (start 114.279377 69.31) (end 114.33 69.31) (width 0.6) (layer B.Cu) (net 15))
 (segment (start 111.76 55.88) (end 111.76 64.74) (width 0.6) (layer B.Cu) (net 16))
 (segment (start 111.76 64.74) (end 114.33 67.31) (width 0.6) (layer B.Cu) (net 16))
 (segment (start 123.19 101.48) (end 123.19 107.95) (width 0.6) (layer B.Cu) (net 13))
 (segment (start 113.87293 107.95) (end 102.44293 96.52) (width 0.6) (layer B.Cu) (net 13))
 (segment (start 120.41 98.7) (end 123.19 101.48) (width 0.6) (layer B.Cu) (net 13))
 (segment (start 120.41 98.45) (end 120.41 98.7) (width 0.6) (layer B.Cu) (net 13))
 (segment (start 94.835002 96.52) (end 93.265001 94.949999) (width 0.6) (layer B.Cu) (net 13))
 (segment (start 123.19 107.95) (end 113.87293 107.95) (width 0.6) (layer B.Cu) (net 13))
 (segment (start 102.44293 96.52) (end 94.835002 96.52) (width 0.6) (layer B.Cu) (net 13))
 (segment (start 104.14 92.71) (end 111.780001 100.350001) (width 0.6) (layer B.Cu) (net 13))
 (segment (start 111.780001 100.350001) (end 120.109999 100.350001) (width 0.6) (layer B.Cu) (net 13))
 (segment (start 120.109999 100.350001) (end 120.41 100.05) (width 0.6) (layer B.Cu) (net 13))
 (segment (start 120.41 100.05) (end 120.41 98.45) (width 0.6) (layer B.Cu) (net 13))
 (segment (start 124.880001 92.289999) (end 125.73 91.44) (width 0.6) (layer B.Cu) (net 13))
 (segment (start 120.41 98.45) (end 120.41 96.76) (width 0.6) (layer B.Cu) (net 13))
 (segment (start 120.41 96.76) (end 124.880001 92.289999) (width 0.6) (layer B.Cu) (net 13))
 (segment (start 91.44 95.25) (end 92.965 95.25) (width 0.6) (layer B.Cu) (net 13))
 (segment (start 92.965 95.25) (end 93.265001 94.949999) (width 0.6) (layer B.Cu) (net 13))
 (segment (start 93.265001 94.949999) (end 93.265001 85.645001) (width 0.6) (layer B.Cu) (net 13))
 (segment (start 93.265001 85.645001) (end 92.289999 84.669999) (width 0.6) (layer B.Cu) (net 13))
 (segment (start 92.289999 84.669999) (end 91.44 83.82) (width 0.6) (layer B.Cu) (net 13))
 (segment (start 100.33 85.09) (end 101.129999 84.290001) (width 0.6) (layer B.Cu) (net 20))
 (segment (start 101.129999 84.290001) (end 101.129999 84.266003) (width 0.6) (layer B.Cu) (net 20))
 (segment (start 102.87 82.526002) (end 102.87 72.413998) (width 0.6) (layer B.Cu) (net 20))
 (segment (start 102.87 72.413998) (end 101.766002 71.31) (width 0.6) (layer B.Cu) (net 20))
 (segment (start 101.129999 84.266003) (end 102.87 82.526002) (width 0.6) (layer B.Cu) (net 20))
 (segment (start 101.766002 71.31) (end 100.33 71.31) (width 0.6) (layer B.Cu) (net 20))
 (segment (start 114.33 79.31) (end 117.41 79.31) (width 0.6) (layer B.Cu) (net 21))
 (segment (start 117.41 79.31) (end 119.38 81.28) (width 0.6) (layer B.Cu) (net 21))
 (segment (start 114.33 75.31) (end 117.73 75.31) (width 0.6) (layer B.Cu) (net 19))
 (segment (start 117.73 75.31) (end 119.38 73.66) (width 0.6) (layer B.Cu) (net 19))
 (segment (start 113.61 86.36) (end 112.610001 85.360001) (width 0.6) (layer B.Cu) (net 19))
 (segment (start 112.610001 85.360001) (end 112.610001 76.979376) (width 0.6) (layer B.Cu) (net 19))
 (segment (start 112.610001 76.979376) (end 114.279377 75.31) (width 0.6) (layer B.Cu) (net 19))
 (segment (start 114.279377 75.31) (end 114.33 75.31) (width 0.6) (layer B.Cu) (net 19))
 (segment (start 114.33 77.31) (end 119.22 77.31) (width 0.6) (layer B.Cu) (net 22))
 (segment (start 119.22 77.31) (end 119.38 77.47) (width 0.6) (layer B.Cu) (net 22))
 (segment (start 91.44 102.87) (end 98.29 102.87) (width 1.2) (layer B.Cu) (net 1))
 (segment (start 98.29 102.87) (end 98.33 102.91) (width 0.6) (layer B.Cu) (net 1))
 (segment (start 91.44 107.95) (end 98.29 107.95) (width 1.2) (layer B.Cu) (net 2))
 (segment (start 98.29 107.95) (end 98.33 107.91) (width 0.6) (layer B.Cu) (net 2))
 (segment (start 112.697999 90.959999) (end 110.947998 92.71) (width 0.6) (layer B.Cu) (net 6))
 (segment (start 110.35137 92.71) (end 109.22 92.71) (width 0.6) (layer B.Cu) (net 6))
 (segment (start 110.947998 92.71) (end 110.35137 92.71) (width 0.6) (layer B.Cu) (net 6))
 (segment (start 128.27 87.63) (end 123.057143 87.63) (width 0.6) (layer B.Cu) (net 6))
 (segment (start 119.727144 90.959999) (end 112.697999 90.959999) (width 0.6) (layer B.Cu) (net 6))
 (segment (start 123.057143 87.63) (end 119.727144 90.959999) (width 0.6) (layer B.Cu) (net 6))
 (segment (start 127.73 113.11) (end 124.46 109.84) (width 0.6) (layer B.Cu) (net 4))
 (segment (start 124.46 109.84) (end 124.46 96.7) (width 0.6) (layer B.Cu) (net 4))
 (segment (start 124.46 96.7) (end 128.27 92.89) (width 0.6) (layer B.Cu) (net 4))
 (segment (start 128.27 92.89) (end 128.27 91.44) (width 0.6) (layer B.Cu) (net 4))
 (segment (start 87.63 69.85) (end 91.44 66.04) (width 0.6) (layer B.Cu) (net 7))
 (segment (start 91.44 66.04) (end 99.06 66.04) (width 0.6) (layer B.Cu) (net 7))
 (segment (start 99.06 66.04) (end 100.33 67.31) (width 0.6) (layer B.Cu) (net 7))
 (segment (start 91.44 66.04) (end 95.25 62.23) (width 0.6) (layer B.Cu) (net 7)))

